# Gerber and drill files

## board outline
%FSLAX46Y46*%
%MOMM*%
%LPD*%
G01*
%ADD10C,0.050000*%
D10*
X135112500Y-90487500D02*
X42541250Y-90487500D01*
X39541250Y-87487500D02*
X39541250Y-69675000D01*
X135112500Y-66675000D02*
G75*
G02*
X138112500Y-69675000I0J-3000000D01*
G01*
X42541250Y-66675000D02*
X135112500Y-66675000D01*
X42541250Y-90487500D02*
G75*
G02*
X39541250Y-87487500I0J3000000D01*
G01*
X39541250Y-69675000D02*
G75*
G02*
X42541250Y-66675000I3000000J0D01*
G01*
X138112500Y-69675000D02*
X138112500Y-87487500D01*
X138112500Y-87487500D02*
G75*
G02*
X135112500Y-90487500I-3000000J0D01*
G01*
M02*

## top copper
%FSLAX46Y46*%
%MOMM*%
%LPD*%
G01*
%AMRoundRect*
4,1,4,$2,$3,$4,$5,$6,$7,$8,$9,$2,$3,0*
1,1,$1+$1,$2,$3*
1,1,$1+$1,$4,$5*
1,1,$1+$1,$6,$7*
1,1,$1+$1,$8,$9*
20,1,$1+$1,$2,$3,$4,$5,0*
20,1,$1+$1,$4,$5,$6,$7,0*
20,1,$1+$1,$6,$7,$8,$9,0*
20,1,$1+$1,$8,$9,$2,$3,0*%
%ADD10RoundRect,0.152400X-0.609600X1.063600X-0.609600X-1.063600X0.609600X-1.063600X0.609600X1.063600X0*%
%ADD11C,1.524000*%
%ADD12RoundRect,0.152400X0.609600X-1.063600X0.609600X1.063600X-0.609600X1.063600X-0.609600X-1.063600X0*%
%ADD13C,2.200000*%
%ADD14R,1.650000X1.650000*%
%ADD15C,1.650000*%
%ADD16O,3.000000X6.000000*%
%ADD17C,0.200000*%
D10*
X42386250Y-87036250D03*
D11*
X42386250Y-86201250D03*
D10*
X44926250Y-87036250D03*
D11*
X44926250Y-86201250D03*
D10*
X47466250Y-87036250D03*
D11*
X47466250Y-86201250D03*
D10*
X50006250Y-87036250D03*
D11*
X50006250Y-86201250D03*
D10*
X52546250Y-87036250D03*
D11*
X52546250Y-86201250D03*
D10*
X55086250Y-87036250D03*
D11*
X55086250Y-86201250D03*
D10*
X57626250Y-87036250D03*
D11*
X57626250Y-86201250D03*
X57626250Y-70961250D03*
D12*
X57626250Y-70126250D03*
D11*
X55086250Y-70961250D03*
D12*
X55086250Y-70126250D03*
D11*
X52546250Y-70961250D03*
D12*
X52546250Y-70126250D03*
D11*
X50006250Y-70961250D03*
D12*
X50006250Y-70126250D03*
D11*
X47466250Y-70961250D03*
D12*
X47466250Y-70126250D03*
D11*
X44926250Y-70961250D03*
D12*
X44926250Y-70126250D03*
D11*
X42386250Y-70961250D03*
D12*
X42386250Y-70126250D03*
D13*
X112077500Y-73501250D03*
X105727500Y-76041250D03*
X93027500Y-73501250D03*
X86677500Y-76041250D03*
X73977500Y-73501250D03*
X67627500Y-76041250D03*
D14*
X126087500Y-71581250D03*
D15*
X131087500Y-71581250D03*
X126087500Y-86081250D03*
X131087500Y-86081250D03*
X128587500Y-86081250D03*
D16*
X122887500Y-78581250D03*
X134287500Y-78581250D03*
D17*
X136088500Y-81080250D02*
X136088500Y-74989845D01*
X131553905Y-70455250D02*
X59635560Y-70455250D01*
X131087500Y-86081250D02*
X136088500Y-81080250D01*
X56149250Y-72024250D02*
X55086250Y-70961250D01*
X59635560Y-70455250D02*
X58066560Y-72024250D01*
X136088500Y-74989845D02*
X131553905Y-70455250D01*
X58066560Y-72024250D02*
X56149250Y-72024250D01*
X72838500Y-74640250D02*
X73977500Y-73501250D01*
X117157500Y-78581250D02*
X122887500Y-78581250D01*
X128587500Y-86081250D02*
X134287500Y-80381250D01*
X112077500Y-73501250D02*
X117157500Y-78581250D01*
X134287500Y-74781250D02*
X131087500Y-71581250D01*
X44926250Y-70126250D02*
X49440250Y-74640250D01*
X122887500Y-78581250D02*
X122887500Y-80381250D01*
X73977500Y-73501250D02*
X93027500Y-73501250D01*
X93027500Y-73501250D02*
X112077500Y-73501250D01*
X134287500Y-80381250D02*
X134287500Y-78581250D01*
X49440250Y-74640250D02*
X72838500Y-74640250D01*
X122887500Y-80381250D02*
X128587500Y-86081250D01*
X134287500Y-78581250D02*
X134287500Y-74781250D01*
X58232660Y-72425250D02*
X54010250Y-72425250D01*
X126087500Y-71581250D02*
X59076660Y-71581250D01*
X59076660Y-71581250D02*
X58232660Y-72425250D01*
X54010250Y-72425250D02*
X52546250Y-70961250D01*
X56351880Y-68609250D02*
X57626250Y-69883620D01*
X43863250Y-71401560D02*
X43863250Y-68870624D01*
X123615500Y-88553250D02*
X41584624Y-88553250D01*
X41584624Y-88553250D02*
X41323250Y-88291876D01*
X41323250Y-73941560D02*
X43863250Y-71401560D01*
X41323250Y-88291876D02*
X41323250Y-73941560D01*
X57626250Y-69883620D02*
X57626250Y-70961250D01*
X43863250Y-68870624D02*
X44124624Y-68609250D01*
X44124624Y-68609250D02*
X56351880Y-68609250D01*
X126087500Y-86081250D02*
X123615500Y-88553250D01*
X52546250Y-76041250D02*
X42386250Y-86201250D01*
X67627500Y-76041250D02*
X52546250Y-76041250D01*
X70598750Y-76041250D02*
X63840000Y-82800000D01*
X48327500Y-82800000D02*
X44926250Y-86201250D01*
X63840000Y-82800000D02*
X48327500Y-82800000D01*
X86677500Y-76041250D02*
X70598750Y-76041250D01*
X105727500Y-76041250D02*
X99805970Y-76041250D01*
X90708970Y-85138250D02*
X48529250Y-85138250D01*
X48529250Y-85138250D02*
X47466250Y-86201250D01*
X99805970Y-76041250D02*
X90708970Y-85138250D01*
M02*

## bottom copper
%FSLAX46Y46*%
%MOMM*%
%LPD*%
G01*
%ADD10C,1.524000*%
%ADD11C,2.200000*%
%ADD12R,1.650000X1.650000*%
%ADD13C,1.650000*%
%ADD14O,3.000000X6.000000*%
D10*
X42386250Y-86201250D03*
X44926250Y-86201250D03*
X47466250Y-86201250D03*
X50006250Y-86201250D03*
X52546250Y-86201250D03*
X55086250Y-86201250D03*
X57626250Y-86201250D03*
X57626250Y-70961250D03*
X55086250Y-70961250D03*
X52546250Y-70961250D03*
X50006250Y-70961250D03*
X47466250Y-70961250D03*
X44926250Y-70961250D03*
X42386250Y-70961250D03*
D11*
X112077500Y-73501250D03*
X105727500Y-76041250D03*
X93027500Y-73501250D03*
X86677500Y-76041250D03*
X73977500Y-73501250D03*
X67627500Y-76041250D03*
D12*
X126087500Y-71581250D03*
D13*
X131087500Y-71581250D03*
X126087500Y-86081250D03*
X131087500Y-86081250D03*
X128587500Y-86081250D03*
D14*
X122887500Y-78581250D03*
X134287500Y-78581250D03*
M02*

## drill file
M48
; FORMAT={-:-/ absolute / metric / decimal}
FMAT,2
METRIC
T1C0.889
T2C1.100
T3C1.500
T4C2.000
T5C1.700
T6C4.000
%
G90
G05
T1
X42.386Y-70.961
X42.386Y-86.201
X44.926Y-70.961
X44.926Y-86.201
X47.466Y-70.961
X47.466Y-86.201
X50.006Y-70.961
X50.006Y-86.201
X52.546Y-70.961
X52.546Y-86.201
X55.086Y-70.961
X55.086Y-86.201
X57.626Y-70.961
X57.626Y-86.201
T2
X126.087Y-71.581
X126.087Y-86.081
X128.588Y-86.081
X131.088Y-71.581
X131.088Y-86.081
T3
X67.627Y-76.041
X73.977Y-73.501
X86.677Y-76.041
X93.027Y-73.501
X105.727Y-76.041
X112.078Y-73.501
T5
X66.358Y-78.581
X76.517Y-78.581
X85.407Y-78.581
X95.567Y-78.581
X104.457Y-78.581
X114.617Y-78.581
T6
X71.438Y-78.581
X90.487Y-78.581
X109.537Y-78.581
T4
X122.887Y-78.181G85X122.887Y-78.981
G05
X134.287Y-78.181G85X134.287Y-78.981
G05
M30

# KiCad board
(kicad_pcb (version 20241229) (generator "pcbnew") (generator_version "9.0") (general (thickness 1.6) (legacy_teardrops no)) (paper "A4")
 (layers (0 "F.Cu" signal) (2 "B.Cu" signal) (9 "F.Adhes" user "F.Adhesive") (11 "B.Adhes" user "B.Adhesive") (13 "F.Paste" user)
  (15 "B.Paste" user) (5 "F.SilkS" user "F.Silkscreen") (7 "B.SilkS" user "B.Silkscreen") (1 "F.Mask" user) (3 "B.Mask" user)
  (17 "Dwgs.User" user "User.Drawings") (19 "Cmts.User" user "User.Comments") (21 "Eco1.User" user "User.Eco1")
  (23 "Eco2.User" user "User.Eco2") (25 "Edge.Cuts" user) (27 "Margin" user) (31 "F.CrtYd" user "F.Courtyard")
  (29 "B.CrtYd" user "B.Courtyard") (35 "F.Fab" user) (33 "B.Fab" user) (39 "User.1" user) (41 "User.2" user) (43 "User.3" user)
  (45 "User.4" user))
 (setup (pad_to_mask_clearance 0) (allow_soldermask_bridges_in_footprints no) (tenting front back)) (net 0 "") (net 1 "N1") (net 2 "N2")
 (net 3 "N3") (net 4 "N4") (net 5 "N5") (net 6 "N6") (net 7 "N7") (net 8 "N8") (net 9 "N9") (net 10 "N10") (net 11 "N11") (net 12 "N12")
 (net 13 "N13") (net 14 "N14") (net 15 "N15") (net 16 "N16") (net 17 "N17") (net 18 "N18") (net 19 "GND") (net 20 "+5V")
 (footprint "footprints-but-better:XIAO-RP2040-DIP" (layer "F.Cu") (at 50.00625 78.58125 90)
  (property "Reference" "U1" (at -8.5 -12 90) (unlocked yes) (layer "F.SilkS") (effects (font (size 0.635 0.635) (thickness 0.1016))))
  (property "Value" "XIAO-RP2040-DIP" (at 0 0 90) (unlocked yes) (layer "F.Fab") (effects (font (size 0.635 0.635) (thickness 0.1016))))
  (pad "1" smd roundrect (at -8.455 -7.62 270) (size 2.432 1.524) (layers "F.Cu" "F.Mask") (roundrect_rratio 0.1) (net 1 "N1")
   (thermal_bridge_angle 45))
  (pad "1" thru_hole circle (at -7.62 -7.62 270) (size 1.524 1.524) (drill 0.889) (layers "*.Cu" "*.Mask") (remove_unused_layers no)
   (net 1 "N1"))
  (pad "2" smd roundrect (at -8.455 -5.08 270) (size 2.432 1.524) (layers "F.Cu" "F.Mask") (roundrect_rratio 0.1) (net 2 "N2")
   (thermal_bridge_angle 45))
  (pad "2" thru_hole circle (at -7.62 -5.08 270) (size 1.524 1.524) (drill 0.889) (layers "*.Cu" "*.Mask") (remove_unused_layers no)
   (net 2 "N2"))
  (pad "3" smd roundrect (at -8.455 -2.54 270) (size 2.432 1.524) (layers "F.Cu" "F.Mask") (roundrect_rratio 0.1) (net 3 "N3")
   (thermal_bridge_angle 45))
  (pad "3" thru_hole circle (at -7.62 -2.54 270) (size 1.524 1.524) (drill 0.889) (layers "*.Cu" "*.Mask") (remove_unused_layers no)
   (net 3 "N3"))
  (pad "4" smd roundrect (at -8.455 0 270) (size 2.432 1.524) (layers "F.Cu" "F.Mask") (roundrect_rratio 0.1) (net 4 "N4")
   (thermal_bridge_angle 45))
  (pad "4" thru_hole circle (at -7.62 0 270) (size 1.524 1.524) (drill 0.889) (layers "*.Cu" "*.Mask") (remove_unused_layers no)
   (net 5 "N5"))
  (pad "5" smd roundrect (at -8.455 2.54 270) (size 2.432 1.524) (layers "F.Cu" "F.Mask") (roundrect_rratio 0.1) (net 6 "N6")
   (thermal_bridge_angle 45))
  (pad "5" thru_hole circle (at -7.62 2.54 270) (size 1.524 1.524) (drill 0.889) (layers "*.Cu" "*.Mask") (remove_unused_layers no)
   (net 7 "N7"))
  (pad "6" smd roundrect (at -8.455 5.08 270) (size 2.432 1.524) (layers "F.Cu" "F.Mask") (roundrect_rratio 0.1) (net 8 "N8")
   (thermal_bridge_angle 45))
  (pad "6" thru_hole circle (at -7.62 5.08 270) (size 1.524 1.524) (drill 0.889) (layers "*.Cu" "*.Mask") (remove_unused_layers no)
   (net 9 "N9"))
  (pad "7" smd roundrect (at -8.455 7.62 270) (size 2.432 1.524) (layers "F.Cu" "F.Mask") (roundrect_rratio 0.1) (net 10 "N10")
   (thermal_bridge_angle 45))
  (pad "7" thru_hole circle (at -7.62 7.62 270) (size 1.524 1.524) (drill 0.889) (layers "*.Cu" "*.Mask") (remove_unused_layers no)
   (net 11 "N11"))
  (pad "8" thru_hole circle (at 7.62 7.62 90) (size 1.524 1.524) (drill 0.889) (layers "*.Cu" "*.Mask") (remove_unused_layers no)
   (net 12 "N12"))
  (pad "8" smd roundrect (at 8.455 7.62 90) (size 2.432 1.524) (layers "F.Cu" "F.Mask") (roundrect_rratio 0.1) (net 12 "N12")
   (thermal_bridge_angle 45))
  (pad "9" thru_hole circle (at 7.62 5.08 90) (size 1.524 1.524) (drill 0.889) (layers "*.Cu" "*.Mask") (remove_unused_layers no)
   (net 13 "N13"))
  (pad "9" smd roundrect (at 8.455 5.08 90) (size 2.432 1.524) (layers "F.Cu" "F.Mask") (roundrect_rratio 0.1) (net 13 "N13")
   (thermal_bridge_angle 45))
  (pad "10" thru_hole circle (at 7.62 2.54 90) (size 1.524 1.524) (drill 0.889) (layers "*.Cu" "*.Mask") (remove_unused_layers no)
   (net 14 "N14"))
  (pad "10" smd roundrect (at 8.455 2.54 90) (size 2.432 1.524) (layers "F.Cu" "F.Mask") (roundrect_rratio 0.1) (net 14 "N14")
   (thermal_bridge_angle 45))
  (pad "11" thru_hole circle (at 7.62 0 90) (size 1.524 1.524) (drill 0.889) (layers "*.Cu" "*.Mask") (remove_unused_layers no)
   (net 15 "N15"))
  (pad "11" smd roundrect (at 8.455 0 90) (size 2.432 1.524) (layers "F.Cu" "F.Mask") (roundrect_rratio 0.1) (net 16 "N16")
   (thermal_bridge_angle 45))
  (pad "12" thru_hole circle (at 7.62 -2.54 90) (size 1.524 1.524) (drill 0.889) (layers "*.Cu" "*.Mask") (remove_unused_layers no)
   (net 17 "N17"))
  (pad "12" smd roundrect (at 8.455 -2.54 90) (size 2.432 1.524) (layers "F.Cu" "F.Mask") (roundrect_rratio 0.1) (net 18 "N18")
   (thermal_bridge_angle 45))
  (pad "13" thru_hole circle (at 7.62 -5.08 90) (size 1.524 1.524) (drill 0.889) (layers "*.Cu" "*.Mask") (remove_unused_layers no)
   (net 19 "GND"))
  (pad "13" smd roundrect (at 8.455 -5.08 90) (size 2.432 1.524) (layers "F.Cu" "F.Mask") (roundrect_rratio 0.1) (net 19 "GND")
   (thermal_bridge_angle 45))
  (pad "14" thru_hole circle (at 7.62 -7.62 90) (size 1.524 1.524) (drill 0.889) (layers "*.Cu" "*.Mask") (remove_unused_layers no)
   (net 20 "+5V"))
  (pad "14" smd roundrect (at 8.455 -7.62 90) (size 2.432 1.524) (layers "F.Cu" "F.Mask") (roundrect_rratio 0.1) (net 20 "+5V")
   (thermal_bridge_angle 45)))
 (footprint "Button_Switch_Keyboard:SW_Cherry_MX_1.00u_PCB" (layer "F.Cu") (at 112.0775 73.50125)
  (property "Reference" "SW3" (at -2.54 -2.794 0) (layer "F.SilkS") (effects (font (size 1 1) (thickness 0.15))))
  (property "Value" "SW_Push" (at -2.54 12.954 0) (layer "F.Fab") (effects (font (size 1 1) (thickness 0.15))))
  (pad "" np_thru_hole circle (at -7.62 5.08) (size 1.7 1.7) (drill 1.7) (layers "*.Cu" "*.Mask"))
  (pad "" np_thru_hole circle (at -2.54 5.08) (size 4 4) (drill 4) (layers "*.Cu" "*.Mask"))
  (pad "" np_thru_hole circle (at 2.54 5.08) (size 1.7 1.7) (drill 1.7) (layers "*.Cu" "*.Mask"))
  (pad "1" thru_hole circle (at 0 0) (size 2.2 2.2) (drill 1.5) (layers "*.Cu" "*.Mask") (remove_unused_layers no) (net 19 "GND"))
  (pad "2" thru_hole circle (at -6.35 2.54) (size 2.2 2.2) (drill 1.5) (layers "*.Cu" "*.Mask") (remove_unused_layers no) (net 3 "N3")))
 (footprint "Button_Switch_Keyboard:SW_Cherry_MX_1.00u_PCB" (layer "F.Cu") (at 93.0275 73.50125)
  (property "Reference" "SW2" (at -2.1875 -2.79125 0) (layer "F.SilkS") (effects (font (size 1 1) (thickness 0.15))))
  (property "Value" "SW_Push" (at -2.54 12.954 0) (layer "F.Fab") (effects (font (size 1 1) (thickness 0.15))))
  (pad "" np_thru_hole circle (at -7.62 5.08) (size 1.7 1.7) (drill 1.7) (layers "*.Cu" "*.Mask"))
  (pad "" np_thru_hole circle (at -2.54 5.08) (size 4 4) (drill 4) (layers "*.Cu" "*.Mask"))
  (pad "" np_thru_hole circle (at 2.54 5.08) (size 1.7 1.7) (drill 1.7) (layers "*.Cu" "*.Mask"))
  (pad "1" thru_hole circle (at 0 0) (size 2.2 2.2) (drill 1.5) (layers "*.Cu" "*.Mask") (remove_unused_layers no) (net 19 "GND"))
  (pad "2" thru_hole circle (at -6.35 2.54) (size 2.2 2.2) (drill 1.5) (layers "*.Cu" "*.Mask") (remove_unused_layers no) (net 2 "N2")))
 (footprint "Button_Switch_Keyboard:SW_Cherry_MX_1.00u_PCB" (layer "F.Cu") (at 73.9775 73.50125)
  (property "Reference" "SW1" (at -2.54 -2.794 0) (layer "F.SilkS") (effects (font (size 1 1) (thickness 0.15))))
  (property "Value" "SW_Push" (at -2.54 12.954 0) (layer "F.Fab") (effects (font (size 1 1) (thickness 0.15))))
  (pad "" np_thru_hole circle (at -7.62 5.08) (size 1.7 1.7) (drill 1.7) (layers "*.Cu" "*.Mask"))
  (pad "" np_thru_hole circle (at -2.54 5.08) (size 4 4) (drill 4) (layers "*.Cu" "*.Mask"))
  (pad "" np_thru_hole circle (at 2.54 5.08) (size 1.7 1.7) (drill 1.7) (layers "*.Cu" "*.Mask"))
  (pad "1" thru_hole circle (at 0 0) (size 2.2 2.2) (drill 1.5) (layers "*.Cu" "*.Mask") (remove_unused_layers no) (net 19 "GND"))
  (pad "2" thru_hole circle (at -6.35 2.54) (size 2.2 2.2) (drill 1.5) (layers "*.Cu" "*.Mask") (remove_unused_layers no) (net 1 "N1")))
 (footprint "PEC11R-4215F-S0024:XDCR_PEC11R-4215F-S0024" (layer "F.Cu") (at 128.5875 78.58125)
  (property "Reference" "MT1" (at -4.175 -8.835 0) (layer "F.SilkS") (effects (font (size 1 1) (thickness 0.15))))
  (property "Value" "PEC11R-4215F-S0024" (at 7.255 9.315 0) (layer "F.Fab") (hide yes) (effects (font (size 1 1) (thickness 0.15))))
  (pad "1" thru_hole rect (at -2.5 -7) (size 1.65 1.65) (drill 1.1) (layers "*.Cu" "*.Mask") (remove_unused_layers no) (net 14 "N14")
   (solder_mask_margin 0.102))
  (pad "2" thru_hole circle (at 2.5 -7) (size 1.65 1.65) (drill 1.1) (layers "*.Cu" "*.Mask") (remove_unused_layers no) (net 19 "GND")
   (solder_mask_margin 0.102))
  (pad "A" thru_hole circle (at -2.5 7.5) (size 1.65 1.65) (drill 1.1) (layers "*.Cu" "*.Mask") (remove_unused_layers no) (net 12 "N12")
   (solder_mask_margin 0.102))
  (pad "B" thru_hole circle (at 2.5 7.5) (size 1.65 1.65) (drill 1.1) (layers "*.Cu" "*.Mask") (remove_unused_layers no) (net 13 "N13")
   (solder_mask_margin 0.102))
  (pad "COM" thru_hole circle (at 0 7.5) (size 1.65 1.65) (drill 1.1) (layers "*.Cu" "*.Mask") (remove_unused_layers no) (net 19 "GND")
   (solder_mask_margin 0.102))
  (pad "S1" thru_hole oval (at -5.7 0) (size 3 6) (drill oval 2 2.8) (layers "*.Cu" "*.Mask") (remove_unused_layers no) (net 19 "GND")
   (solder_mask_margin 0.102))
  (pad "S2" thru_hole oval (at 5.7 0) (size 3 6) (drill oval 2 2.8) (layers "*.Cu" "*.Mask") (remove_unused_layers no) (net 19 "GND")
   (solder_mask_margin 0.102)))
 (gr_line (start 135.1125 90.4875) (end 42.54125 90.4875) (stroke (width 0.05) (type default)) (layer "Edge.Cuts"))
 (gr_line (start 39.54125 87.4875) (end 39.54125 69.675) (stroke (width 0.05) (type default)) (layer "Edge.Cuts"))
 (gr_arc (start 135.1125 66.675) (mid 137.23382 67.55368) (end 138.1125 69.675) (stroke (width 0.05) (type default)) (layer "Edge.Cuts"))
 (gr_line (start 42.54125 66.675) (end 135.1125 66.675) (stroke (width 0.05) (type default)) (layer "Edge.Cuts"))
 (gr_arc (start 42.54125 90.4875) (mid 40.41993 89.60882) (end 39.54125 87.4875) (stroke (width 0.05) (type default)) (layer "Edge.Cuts"))
 (gr_arc (start 39.54125 69.675) (mid 40.41993 67.55368) (end 42.54125 66.675) (stroke (width 0.05) (type default)) (layer "Edge.Cuts"))
 (gr_line (start 138.1125 69.675) (end 138.1125 87.4875) (stroke (width 0.05) (type default)) (layer "Edge.Cuts"))
 (gr_arc (start 138.1125 87.4875) (mid 137.23382 89.60882) (end 135.1125 90.4875) (stroke (width 0.05) (type default)) (layer "Edge.Cuts"))
 (segment (start 136.0885 81.08025) (end 136.0885 74.989845) (width 0.2) (layer "F.Cu") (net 13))
 (segment (start 131.553905 70.45525) (end 59.63556 70.45525) (width 0.2) (layer "F.Cu") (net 13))
 (segment (start 131.0875 86.08125) (end 136.0885 81.08025) (width 0.2) (layer "F.Cu") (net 13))
 (segment (start 56.14925 72.02425) (end 55.08625 70.96125) (width 0.2) (layer "F.Cu") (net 13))
 (segment (start 59.63556 70.45525) (end 58.06656 72.02425) (width 0.2) (layer "F.Cu") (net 13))
 (segment (start 136.0885 74.989845) (end 131.553905 70.45525) (width 0.2) (layer "F.Cu") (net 13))
 (segment (start 58.06656 72.02425) (end 56.14925 72.02425) (width 0.2) (layer "F.Cu") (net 13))
 (segment (start 72.8385 74.64025) (end 73.9775 73.50125) (width 0.2) (layer "F.Cu") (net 19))
 (segment (start 117.1575 78.58125) (end 122.8875 78.58125) (width 0.2) (layer "F.Cu") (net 19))
 (segment (start 128.5875 86.08125) (end 134.2875 80.38125) (width 0.2) (layer "F.Cu") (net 19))
 (segment (start 112.0775 73.50125) (end 117.1575 78.58125) (width 0.2) (layer "F.Cu") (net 19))
 (segment (start 134.2875 74.78125) (end 131.0875 71.58125) (width 0.2) (layer "F.Cu") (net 19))
 (segment (start 44.92625 70.12625) (end 49.44025 74.64025) (width 0.2) (layer "F.Cu") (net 19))
 (segment (start 122.8875 78.58125) (end 122.8875 80.38125) (width 0.2) (layer "F.Cu") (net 19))
 (segment (start 73.9775 73.50125) (end 93.0275 73.50125) (width 0.2) (layer "F.Cu") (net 19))
 (segment (start 93.0275 73.50125) (end 112.0775 73.50125) (width 0.2) (layer "F.Cu") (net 19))
 (segment (start 134.2875 80.38125) (end 134.2875 78.58125) (width 0.2) (layer "F.Cu") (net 19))
 (segment (start 49.44025 74.64025) (end 72.8385 74.64025) (width 0.2) (layer "F.Cu") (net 19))
 (segment (start 122.8875 80.38125) (end 128.5875 86.08125) (width 0.2) (layer "F.Cu") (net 19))
 (segment (start 134.2875 78.58125) (end 134.2875 74.78125) (width 0.2) (layer "F.Cu") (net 19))
 (segment (start 58.23266 72.42525) (end 54.01025 72.42525) (width 0.2) (layer "F.Cu") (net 14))
 (segment (start 126.0875 71.58125) (end 59.07666 71.58125) (width 0.2) (layer "F.Cu") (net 14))
 (segment (start 59.07666 71.58125) (end 58.23266 72.42525) (width 0.2) (layer "F.Cu") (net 14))
 (segment (start 54.01025 72.42525) (end 52.54625 70.96125) (width 0.2) (layer "F.Cu") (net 14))
 (segment (start 56.35188 68.60925) (end 57.62625 69.88362) (width 0.2) (layer "F.Cu") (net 12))
 (segment (start 43.86325 71.40156) (end 43.86325 68.870624) (width 0.2) (layer "F.Cu") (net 12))
 (segment (start 123.6155 88.55325) (end 41.584624 88.55325) (width 0.2) (layer "F.Cu") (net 12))
 (segment (start 41.584624 88.55325) (end 41.32325 88.291876) (width 0.2) (layer "F.Cu") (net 12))
 (segment (start 41.32325 73.94156) (end 43.86325 71.40156) (width 0.2) (layer "F.Cu") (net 12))
 (segment (start 41.32325 88.291876) (end 41.32325 73.94156) (width 0.2) (layer "F.Cu") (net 12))
 (segment (start 57.62625 69.88362) (end 57.62625 70.96125) (width 0.2) (layer "F.Cu") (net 12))
 (segment (start 43.86325 68.870624) (end 44.124624 68.60925) (width 0.2) (layer "F.Cu") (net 12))
 (segment (start 44.124624 68.60925) (end 56.35188 68.60925) (width 0.2) (layer "F.Cu") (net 12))
 (segment (start 126.0875 86.08125) (end 123.6155 88.55325) (width 0.2) (layer "F.Cu") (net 12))
 (segment (start 52.54625 76.04125) (end 42.38625 86.20125) (width 0.2) (layer "F.Cu") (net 1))
 (segment (start 67.6275 76.04125) (end 52.54625 76.04125) (width 0.2) (layer "F.Cu") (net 1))
 (segment (start 70.59875 76.04125) (end 63.84 82.8) (width 0.2) (layer "F.Cu") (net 2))
 (segment (start 48.3275 82.8) (end 44.92625 86.20125) (width 0.2) (layer "F.Cu") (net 2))
 (segment (start 63.84 82.8) (end 48.3275 82.8) (width 0.2) (layer "F.Cu") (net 2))
 (segment (start 86.6775 76.04125) (end 70.59875 76.04125) (width 0.2) (layer "F.Cu") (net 2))
 (segment (start 105.7275 76.04125) (end 99.80597 76.04125) (width 0.2) (layer "F.Cu") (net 3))
 (segment (start 90.70897 85.13825) (end 48.52925 85.13825) (width 0.2) (layer "F.Cu") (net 3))
 (segment (start 48.52925 85.13825) (end 47.46625 86.20125) (width 0.2) (layer "F.Cu") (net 3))
 (segment (start 99.80597 76.04125) (end 90.70897 85.13825) (width 0.2) (layer "F.Cu") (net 3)))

